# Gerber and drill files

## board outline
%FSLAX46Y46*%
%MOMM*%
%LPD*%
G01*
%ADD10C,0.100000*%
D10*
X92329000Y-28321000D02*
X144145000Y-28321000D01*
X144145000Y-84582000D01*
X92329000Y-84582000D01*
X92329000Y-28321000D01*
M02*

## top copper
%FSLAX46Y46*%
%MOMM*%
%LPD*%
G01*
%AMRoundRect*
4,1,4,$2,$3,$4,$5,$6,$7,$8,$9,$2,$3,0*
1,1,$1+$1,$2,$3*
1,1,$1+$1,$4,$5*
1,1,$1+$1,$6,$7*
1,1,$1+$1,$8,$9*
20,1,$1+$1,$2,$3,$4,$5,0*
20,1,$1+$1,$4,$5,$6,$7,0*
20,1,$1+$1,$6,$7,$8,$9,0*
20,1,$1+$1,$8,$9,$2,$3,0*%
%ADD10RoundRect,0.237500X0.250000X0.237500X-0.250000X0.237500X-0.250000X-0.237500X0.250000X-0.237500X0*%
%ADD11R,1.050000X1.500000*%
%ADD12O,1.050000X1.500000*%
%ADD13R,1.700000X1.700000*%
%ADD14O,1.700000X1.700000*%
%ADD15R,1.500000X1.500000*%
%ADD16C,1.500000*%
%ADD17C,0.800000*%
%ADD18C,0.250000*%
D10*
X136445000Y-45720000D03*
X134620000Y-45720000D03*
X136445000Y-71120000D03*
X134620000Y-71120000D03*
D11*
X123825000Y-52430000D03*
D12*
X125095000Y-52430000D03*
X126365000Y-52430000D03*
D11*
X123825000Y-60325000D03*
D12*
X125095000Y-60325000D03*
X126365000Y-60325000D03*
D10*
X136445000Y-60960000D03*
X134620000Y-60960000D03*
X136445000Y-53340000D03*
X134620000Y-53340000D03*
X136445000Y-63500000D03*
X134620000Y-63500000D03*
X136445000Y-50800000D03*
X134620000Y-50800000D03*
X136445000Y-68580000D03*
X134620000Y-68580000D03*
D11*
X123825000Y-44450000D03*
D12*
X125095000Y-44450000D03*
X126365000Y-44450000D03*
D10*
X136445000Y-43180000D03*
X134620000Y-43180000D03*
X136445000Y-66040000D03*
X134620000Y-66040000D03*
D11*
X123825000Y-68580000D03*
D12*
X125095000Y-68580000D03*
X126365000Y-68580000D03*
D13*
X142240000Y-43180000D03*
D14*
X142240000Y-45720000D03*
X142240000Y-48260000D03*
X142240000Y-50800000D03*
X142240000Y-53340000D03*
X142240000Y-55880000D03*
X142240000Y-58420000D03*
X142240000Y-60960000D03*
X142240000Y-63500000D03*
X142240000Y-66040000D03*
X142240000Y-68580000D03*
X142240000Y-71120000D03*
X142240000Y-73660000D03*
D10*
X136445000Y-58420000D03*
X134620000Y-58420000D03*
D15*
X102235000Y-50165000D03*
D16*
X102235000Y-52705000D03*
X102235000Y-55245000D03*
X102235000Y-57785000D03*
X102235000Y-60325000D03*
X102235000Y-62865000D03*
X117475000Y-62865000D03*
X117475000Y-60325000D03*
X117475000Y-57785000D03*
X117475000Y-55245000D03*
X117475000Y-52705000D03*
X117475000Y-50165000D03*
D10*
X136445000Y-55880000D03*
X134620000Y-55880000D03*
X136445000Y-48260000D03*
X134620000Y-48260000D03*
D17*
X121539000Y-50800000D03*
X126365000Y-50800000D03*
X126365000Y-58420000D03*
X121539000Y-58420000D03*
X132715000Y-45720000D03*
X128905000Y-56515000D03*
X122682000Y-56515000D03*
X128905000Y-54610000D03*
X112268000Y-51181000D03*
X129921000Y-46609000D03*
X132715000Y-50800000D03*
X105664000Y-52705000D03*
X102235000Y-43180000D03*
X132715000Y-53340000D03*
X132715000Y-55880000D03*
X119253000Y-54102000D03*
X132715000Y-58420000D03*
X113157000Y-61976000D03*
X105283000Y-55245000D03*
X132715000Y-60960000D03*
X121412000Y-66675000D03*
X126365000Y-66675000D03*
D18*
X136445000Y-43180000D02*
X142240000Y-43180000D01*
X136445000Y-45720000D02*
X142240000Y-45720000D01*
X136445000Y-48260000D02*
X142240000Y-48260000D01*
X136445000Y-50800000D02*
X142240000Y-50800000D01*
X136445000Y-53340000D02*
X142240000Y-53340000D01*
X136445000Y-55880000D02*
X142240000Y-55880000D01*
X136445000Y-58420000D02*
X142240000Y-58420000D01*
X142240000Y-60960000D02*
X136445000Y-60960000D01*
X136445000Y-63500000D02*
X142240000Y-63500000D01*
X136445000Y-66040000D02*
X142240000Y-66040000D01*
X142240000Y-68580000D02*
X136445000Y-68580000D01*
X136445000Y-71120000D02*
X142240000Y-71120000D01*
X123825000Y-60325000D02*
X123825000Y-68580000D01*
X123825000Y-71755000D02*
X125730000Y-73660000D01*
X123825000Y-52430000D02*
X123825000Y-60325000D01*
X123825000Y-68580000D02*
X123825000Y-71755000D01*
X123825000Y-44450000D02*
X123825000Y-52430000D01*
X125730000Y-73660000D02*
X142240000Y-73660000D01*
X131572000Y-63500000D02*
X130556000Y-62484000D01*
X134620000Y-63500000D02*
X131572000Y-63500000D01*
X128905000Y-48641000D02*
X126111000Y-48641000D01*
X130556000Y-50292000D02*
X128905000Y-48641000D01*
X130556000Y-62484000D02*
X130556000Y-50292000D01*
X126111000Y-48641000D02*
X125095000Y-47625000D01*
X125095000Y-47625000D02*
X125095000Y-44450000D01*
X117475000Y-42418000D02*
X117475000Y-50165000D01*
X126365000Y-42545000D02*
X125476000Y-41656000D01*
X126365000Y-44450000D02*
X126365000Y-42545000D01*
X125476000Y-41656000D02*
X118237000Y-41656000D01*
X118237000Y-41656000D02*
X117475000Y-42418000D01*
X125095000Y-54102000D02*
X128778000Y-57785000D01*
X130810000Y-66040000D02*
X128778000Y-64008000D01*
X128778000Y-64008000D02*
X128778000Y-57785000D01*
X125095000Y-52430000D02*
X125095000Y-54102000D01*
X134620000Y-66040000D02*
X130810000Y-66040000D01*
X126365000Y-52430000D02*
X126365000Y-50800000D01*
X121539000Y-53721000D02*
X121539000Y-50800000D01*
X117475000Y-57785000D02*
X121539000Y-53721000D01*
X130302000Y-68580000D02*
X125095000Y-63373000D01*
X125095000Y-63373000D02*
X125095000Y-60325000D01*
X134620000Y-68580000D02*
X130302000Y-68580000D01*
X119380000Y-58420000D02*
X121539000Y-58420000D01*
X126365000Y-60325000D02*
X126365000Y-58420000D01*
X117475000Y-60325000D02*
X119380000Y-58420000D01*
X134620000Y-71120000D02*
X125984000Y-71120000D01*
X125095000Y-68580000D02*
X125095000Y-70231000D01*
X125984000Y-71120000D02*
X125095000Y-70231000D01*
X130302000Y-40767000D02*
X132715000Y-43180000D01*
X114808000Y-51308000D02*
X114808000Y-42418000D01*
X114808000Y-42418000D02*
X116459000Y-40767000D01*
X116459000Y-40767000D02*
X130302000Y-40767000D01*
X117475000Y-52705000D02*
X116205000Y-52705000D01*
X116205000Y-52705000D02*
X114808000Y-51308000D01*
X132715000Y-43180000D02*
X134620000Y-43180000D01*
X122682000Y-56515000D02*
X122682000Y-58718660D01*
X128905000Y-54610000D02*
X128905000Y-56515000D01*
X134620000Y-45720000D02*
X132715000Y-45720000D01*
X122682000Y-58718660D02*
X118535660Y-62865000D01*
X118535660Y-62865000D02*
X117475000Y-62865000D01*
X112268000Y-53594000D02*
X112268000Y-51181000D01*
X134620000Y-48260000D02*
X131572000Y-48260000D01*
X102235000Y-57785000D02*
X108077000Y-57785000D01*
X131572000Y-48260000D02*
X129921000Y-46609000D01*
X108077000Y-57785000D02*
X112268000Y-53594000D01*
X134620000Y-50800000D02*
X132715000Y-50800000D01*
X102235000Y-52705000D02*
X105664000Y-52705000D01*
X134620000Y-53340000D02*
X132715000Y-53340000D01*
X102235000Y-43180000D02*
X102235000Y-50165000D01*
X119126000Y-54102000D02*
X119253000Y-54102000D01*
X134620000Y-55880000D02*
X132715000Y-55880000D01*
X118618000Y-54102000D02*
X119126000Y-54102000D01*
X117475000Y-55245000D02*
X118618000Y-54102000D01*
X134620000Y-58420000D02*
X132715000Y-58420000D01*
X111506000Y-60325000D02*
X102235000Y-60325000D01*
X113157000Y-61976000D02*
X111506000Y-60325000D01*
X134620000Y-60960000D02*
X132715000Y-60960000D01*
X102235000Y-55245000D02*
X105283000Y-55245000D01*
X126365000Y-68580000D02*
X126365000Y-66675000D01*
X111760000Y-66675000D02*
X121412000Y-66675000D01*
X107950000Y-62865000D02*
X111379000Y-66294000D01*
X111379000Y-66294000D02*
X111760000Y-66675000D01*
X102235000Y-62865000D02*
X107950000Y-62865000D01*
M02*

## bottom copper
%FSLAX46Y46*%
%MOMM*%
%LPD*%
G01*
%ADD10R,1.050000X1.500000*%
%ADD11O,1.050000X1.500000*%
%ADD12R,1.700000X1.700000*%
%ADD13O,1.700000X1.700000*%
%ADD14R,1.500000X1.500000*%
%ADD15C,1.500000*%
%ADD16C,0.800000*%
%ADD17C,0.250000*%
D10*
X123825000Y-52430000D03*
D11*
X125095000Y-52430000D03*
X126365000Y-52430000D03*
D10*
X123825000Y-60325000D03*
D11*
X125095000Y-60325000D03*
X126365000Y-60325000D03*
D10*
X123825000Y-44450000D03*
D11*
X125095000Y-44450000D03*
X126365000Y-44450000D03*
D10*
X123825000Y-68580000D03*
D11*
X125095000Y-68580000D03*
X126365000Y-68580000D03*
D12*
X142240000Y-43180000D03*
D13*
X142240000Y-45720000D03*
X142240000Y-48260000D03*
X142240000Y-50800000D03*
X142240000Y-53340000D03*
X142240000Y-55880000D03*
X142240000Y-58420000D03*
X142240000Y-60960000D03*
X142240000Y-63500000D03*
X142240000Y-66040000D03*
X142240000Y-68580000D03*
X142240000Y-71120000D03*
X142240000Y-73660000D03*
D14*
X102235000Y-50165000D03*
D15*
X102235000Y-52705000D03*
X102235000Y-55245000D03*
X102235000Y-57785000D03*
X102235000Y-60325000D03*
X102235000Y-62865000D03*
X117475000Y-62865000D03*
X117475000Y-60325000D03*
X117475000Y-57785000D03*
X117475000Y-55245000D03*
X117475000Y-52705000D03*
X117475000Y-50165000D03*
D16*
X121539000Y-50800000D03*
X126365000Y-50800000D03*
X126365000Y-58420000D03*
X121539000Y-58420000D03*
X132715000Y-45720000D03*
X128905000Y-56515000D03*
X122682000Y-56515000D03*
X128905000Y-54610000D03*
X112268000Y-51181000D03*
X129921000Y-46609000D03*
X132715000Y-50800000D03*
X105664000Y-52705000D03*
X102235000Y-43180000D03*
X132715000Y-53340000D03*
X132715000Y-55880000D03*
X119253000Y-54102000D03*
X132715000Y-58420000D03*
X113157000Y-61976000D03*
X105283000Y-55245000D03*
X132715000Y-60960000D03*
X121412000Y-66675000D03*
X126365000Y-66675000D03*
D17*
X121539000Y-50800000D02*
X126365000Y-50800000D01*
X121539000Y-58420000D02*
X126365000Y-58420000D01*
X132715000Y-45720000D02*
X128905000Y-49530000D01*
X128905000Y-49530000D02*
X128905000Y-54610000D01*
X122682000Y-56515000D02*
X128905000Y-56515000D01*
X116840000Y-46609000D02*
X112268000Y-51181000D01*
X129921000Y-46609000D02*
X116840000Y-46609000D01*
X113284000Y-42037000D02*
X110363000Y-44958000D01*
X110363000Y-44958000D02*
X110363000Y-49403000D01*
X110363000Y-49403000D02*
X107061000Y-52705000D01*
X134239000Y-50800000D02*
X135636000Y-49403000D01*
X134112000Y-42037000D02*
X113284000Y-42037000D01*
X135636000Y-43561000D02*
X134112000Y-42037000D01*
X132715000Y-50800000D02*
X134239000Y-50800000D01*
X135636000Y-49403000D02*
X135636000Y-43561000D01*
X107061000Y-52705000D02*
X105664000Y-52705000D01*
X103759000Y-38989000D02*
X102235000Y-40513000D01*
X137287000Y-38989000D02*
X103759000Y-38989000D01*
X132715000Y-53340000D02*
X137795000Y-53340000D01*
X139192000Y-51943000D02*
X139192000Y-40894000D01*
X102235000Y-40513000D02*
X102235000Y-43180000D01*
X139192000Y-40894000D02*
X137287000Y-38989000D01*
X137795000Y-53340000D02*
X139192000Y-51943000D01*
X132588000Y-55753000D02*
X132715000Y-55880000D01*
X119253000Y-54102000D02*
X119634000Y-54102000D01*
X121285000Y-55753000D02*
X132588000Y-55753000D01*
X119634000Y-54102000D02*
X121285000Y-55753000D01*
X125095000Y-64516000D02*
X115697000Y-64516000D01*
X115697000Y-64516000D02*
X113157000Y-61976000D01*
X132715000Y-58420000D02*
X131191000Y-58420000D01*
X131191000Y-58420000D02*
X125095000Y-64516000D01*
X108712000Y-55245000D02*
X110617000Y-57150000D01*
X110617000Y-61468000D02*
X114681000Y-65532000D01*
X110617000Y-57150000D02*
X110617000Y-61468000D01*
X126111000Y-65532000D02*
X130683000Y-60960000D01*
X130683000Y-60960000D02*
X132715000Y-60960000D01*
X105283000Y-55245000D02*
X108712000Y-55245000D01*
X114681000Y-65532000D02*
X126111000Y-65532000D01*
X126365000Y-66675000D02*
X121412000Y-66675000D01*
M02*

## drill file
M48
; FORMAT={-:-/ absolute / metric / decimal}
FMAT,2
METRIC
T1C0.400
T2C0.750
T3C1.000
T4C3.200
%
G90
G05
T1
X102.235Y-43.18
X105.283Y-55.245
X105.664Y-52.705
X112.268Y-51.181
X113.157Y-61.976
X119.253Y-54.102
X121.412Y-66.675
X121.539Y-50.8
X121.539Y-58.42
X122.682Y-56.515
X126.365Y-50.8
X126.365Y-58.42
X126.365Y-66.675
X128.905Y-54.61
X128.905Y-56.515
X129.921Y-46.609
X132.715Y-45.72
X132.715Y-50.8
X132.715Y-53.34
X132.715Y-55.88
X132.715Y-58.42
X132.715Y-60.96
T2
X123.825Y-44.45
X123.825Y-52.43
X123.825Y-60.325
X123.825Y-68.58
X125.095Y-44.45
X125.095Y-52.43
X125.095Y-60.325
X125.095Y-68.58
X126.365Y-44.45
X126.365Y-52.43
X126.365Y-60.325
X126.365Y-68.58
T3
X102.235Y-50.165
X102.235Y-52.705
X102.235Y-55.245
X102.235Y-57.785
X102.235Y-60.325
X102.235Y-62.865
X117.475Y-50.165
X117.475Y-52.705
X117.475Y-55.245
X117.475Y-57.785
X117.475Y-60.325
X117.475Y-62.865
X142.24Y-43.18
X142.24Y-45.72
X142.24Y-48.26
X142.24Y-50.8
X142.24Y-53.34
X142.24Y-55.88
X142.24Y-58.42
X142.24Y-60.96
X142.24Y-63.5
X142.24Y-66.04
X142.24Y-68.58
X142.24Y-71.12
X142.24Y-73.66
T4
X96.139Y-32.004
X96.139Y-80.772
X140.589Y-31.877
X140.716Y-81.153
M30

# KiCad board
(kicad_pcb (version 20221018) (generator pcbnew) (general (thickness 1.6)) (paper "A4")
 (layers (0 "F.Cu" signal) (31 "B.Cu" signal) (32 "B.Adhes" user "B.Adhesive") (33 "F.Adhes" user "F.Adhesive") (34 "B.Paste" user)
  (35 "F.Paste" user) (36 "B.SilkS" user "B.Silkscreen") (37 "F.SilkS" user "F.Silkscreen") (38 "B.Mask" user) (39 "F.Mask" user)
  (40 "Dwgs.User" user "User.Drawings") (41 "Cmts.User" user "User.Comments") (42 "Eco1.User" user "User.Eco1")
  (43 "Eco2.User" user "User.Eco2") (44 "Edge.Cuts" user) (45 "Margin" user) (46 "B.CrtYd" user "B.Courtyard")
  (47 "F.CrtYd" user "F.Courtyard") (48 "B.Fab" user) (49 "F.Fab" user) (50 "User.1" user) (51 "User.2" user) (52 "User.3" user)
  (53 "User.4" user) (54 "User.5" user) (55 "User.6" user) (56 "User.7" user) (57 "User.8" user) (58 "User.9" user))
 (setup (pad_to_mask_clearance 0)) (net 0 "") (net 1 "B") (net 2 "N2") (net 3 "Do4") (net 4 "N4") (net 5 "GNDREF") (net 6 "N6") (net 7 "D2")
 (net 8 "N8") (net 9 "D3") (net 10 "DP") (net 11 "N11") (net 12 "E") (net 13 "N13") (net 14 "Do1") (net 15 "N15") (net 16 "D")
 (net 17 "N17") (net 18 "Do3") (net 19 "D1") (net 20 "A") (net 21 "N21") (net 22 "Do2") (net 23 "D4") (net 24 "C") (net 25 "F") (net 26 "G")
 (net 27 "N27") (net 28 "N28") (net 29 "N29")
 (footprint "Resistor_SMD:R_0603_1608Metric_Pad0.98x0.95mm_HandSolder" (layer "F.Cu") (at 135.5325 45.72 180)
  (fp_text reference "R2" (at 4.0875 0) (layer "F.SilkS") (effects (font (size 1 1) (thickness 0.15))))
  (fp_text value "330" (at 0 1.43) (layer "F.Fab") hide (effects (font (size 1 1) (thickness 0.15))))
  (pad "1" smd roundrect (at -0.9125 0 180) (size 0.975 0.95) (layers "F.Cu" "F.Paste" "F.Mask") (roundrect_rratio 0.25) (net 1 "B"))
  (pad "2" smd roundrect (at 0.9125 0 180) (size 0.975 0.95) (layers "F.Cu" "F.Paste" "F.Mask") (roundrect_rratio 0.25) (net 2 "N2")))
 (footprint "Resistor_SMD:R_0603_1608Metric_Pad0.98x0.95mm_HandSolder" (layer "F.Cu") (at 135.5325 71.12 180)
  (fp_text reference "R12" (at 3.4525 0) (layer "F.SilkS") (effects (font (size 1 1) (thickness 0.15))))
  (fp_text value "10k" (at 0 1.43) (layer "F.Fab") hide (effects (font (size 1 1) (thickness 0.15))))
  (pad "1" smd roundrect (at -0.9125 0 180) (size 0.975 0.95) (layers "F.Cu" "F.Paste" "F.Mask") (roundrect_rratio 0.25) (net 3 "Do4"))
  (pad "2" smd roundrect (at 0.9125 0 180) (size 0.975 0.95) (layers "F.Cu" "F.Paste" "F.Mask") (roundrect_rratio 0.25) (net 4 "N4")))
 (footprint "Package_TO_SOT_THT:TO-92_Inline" (layer "F.Cu") (at 123.825 52.43)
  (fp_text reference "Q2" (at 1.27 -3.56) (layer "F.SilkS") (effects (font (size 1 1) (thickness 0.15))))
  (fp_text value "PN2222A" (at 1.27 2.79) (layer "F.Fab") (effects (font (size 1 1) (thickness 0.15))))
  (pad "1" thru_hole rect (at 0 0) (size 1.05 1.5) (drill 0.75) (layers "*.Cu" "*.Mask") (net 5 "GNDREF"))
  (pad "2" thru_hole oval (at 1.27 0) (size 1.05 1.5) (drill 0.75) (layers "*.Cu" "*.Mask") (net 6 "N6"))
  (pad "3" thru_hole oval (at 2.54 0) (size 1.05 1.5) (drill 0.75) (layers "*.Cu" "*.Mask") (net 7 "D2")))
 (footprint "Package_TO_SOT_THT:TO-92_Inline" (layer "F.Cu") (at 123.825 60.325)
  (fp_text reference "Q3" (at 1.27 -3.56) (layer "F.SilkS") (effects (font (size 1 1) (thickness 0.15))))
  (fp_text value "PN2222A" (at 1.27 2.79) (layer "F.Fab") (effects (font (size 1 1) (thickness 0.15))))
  (pad "1" thru_hole rect (at 0 0) (size 1.05 1.5) (drill 0.75) (layers "*.Cu" "*.Mask") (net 5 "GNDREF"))
  (pad "2" thru_hole oval (at 1.27 0) (size 1.05 1.5) (drill 0.75) (layers "*.Cu" "*.Mask") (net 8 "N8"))
  (pad "3" thru_hole oval (at 2.54 0) (size 1.05 1.5) (drill 0.75) (layers "*.Cu" "*.Mask") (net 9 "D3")))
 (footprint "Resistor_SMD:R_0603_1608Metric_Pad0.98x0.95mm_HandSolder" (layer "F.Cu") (at 135.5325 60.96 180)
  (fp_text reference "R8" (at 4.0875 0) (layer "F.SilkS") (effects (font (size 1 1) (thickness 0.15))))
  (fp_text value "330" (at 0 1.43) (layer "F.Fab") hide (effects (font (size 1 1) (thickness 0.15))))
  (pad "1" smd roundrect (at -0.9125 0 180) (size 0.975 0.95) (layers "F.Cu" "F.Paste" "F.Mask") (roundrect_rratio 0.25) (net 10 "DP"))
  (pad "2" smd roundrect (at 0.9125 0 180) (size 0.975 0.95) (layers "F.Cu" "F.Paste" "F.Mask") (roundrect_rratio 0.25) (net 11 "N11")))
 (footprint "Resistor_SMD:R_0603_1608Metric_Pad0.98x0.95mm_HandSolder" (layer "F.Cu") (at 135.5325 53.34 180)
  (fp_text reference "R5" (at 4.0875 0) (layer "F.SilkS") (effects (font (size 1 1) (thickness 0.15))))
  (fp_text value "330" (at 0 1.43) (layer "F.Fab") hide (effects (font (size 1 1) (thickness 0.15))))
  (pad "1" smd roundrect (at -0.9125 0 180) (size 0.975 0.95) (layers "F.Cu" "F.Paste" "F.Mask") (roundrect_rratio 0.25) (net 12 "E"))
  (pad "2" smd roundrect (at 0.9125 0 180) (size 0.975 0.95) (layers "F.Cu" "F.Paste" "F.Mask") (roundrect_rratio 0.25) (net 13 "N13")))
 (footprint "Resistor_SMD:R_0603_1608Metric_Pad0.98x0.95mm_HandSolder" (layer "F.Cu") (at 135.5325 63.5 180)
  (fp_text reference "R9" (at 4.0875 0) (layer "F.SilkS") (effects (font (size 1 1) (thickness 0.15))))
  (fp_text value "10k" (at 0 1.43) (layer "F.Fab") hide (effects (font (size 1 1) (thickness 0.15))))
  (pad "1" smd roundrect (at -0.9125 0 180) (size 0.975 0.95) (layers "F.Cu" "F.Paste" "F.Mask") (roundrect_rratio 0.25) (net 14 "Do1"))
  (pad "2" smd roundrect (at 0.9125 0 180) (size 0.975 0.95) (layers "F.Cu" "F.Paste" "F.Mask") (roundrect_rratio 0.25) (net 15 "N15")))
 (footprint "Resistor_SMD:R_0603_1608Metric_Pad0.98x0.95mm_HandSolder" (layer "F.Cu") (at 135.5325 50.8 180)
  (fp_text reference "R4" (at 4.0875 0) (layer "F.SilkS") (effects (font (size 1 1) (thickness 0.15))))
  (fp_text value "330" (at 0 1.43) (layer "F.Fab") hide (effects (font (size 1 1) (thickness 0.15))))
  (pad "1" smd roundrect (at -0.9125 0 180) (size 0.975 0.95) (layers "F.Cu" "F.Paste" "F.Mask") (roundrect_rratio 0.25) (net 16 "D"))
  (pad "2" smd roundrect (at 0.9125 0 180) (size 0.975 0.95) (layers "F.Cu" "F.Paste" "F.Mask") (roundrect_rratio 0.25) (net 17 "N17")))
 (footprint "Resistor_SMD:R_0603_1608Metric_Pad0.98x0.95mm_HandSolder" (layer "F.Cu") (at 135.5325 68.58 180)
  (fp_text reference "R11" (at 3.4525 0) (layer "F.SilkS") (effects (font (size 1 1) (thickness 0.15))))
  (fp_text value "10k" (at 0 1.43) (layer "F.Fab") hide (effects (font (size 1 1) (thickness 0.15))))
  (pad "1" smd roundrect (at -0.9125 0 180) (size 0.975 0.95) (layers "F.Cu" "F.Paste" "F.Mask") (roundrect_rratio 0.25) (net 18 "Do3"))
  (pad "2" smd roundrect (at 0.9125 0 180) (size 0.975 0.95) (layers "F.Cu" "F.Paste" "F.Mask") (roundrect_rratio 0.25) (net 8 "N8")))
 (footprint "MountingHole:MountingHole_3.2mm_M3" (layer "F.Cu") (at 96.139 32.004)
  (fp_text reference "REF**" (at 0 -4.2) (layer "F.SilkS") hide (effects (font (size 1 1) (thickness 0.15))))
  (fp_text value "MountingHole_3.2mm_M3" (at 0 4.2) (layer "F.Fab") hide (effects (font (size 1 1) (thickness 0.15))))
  (pad "" np_thru_hole circle (at 0 0) (size 3.2 3.2) (drill 3.2) (layers "*.Cu" "*.Mask")))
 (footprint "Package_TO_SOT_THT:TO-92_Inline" (layer "F.Cu") (at 123.825 44.45)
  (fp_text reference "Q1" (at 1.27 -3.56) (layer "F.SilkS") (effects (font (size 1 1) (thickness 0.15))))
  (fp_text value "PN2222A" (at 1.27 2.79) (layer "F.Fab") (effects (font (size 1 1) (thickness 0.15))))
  (pad "1" thru_hole rect (at 0 0) (size 1.05 1.5) (drill 0.75) (layers "*.Cu" "*.Mask") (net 5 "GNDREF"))
  (pad "2" thru_hole oval (at 1.27 0) (size 1.05 1.5) (drill 0.75) (layers "*.Cu" "*.Mask") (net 15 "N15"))
  (pad "3" thru_hole oval (at 2.54 0) (size 1.05 1.5) (drill 0.75) (layers "*.Cu" "*.Mask") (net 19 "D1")))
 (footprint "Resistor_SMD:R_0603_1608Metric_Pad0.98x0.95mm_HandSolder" (layer "F.Cu") (at 135.5325 43.18 180)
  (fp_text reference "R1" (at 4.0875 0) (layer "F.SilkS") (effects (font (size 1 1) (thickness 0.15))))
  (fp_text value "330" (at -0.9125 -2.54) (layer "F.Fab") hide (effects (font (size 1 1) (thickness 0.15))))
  (pad "1" smd roundrect (at -0.9125 0 180) (size 0.975 0.95) (layers "F.Cu" "F.Paste" "F.Mask") (roundrect_rratio 0.25) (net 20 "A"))
  (pad "2" smd roundrect (at 0.9125 0 180) (size 0.975 0.95) (layers "F.Cu" "F.Paste" "F.Mask") (roundrect_rratio 0.25) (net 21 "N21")))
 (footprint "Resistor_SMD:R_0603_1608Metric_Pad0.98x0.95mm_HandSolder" (layer "F.Cu") (at 135.5325 66.04 180)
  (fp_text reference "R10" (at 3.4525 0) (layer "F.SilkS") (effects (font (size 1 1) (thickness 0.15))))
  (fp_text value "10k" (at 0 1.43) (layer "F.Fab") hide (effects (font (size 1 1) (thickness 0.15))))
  (pad "1" smd roundrect (at -0.9125 0 180) (size 0.975 0.95) (layers "F.Cu" "F.Paste" "F.Mask") (roundrect_rratio 0.25) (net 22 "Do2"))
  (pad "2" smd roundrect (at 0.9125 0 180) (size 0.975 0.95) (layers "F.Cu" "F.Paste" "F.Mask") (roundrect_rratio 0.25) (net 6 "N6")))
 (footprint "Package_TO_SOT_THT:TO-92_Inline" (layer "F.Cu") (at 123.825 68.58)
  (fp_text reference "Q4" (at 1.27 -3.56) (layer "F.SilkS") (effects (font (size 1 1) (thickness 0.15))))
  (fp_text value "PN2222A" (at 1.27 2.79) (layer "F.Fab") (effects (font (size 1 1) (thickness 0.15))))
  (pad "1" thru_hole rect (at 0 0) (size 1.05 1.5) (drill 0.75) (layers "*.Cu" "*.Mask") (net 5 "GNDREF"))
  (pad "2" thru_hole oval (at 1.27 0) (size 1.05 1.5) (drill 0.75) (layers "*.Cu" "*.Mask") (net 4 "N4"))
  (pad "3" thru_hole oval (at 2.54 0) (size 1.05 1.5) (drill 0.75) (layers "*.Cu" "*.Mask") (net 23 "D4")))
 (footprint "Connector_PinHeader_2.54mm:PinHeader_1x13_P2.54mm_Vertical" (layer "F.Cu") (at 142.24 43.18)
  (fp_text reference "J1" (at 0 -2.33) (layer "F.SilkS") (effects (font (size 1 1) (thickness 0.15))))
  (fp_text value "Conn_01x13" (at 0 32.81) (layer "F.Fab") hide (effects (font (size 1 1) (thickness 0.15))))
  (pad "1" thru_hole rect (at 0 0) (size 1.7 1.7) (drill 1) (layers "*.Cu" "*.Mask") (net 20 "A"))
  (pad "2" thru_hole oval (at 0 2.54) (size 1.7 1.7) (drill 1) (layers "*.Cu" "*.Mask") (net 1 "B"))
  (pad "3" thru_hole oval (at 0 5.08) (size 1.7 1.7) (drill 1) (layers "*.Cu" "*.Mask") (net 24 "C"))
  (pad "4" thru_hole oval (at 0 7.62) (size 1.7 1.7) (drill 1) (layers "*.Cu" "*.Mask") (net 16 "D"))
  (pad "5" thru_hole oval (at 0 10.16) (size 1.7 1.7) (drill 1) (layers "*.Cu" "*.Mask") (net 12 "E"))
  (pad "6" thru_hole oval (at 0 12.7) (size 1.7 1.7) (drill 1) (layers "*.Cu" "*.Mask") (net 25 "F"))
  (pad "7" thru_hole oval (at 0 15.24) (size 1.7 1.7) (drill 1) (layers "*.Cu" "*.Mask") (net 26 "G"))
  (pad "8" thru_hole oval (at 0 17.78) (size 1.7 1.7) (drill 1) (layers "*.Cu" "*.Mask") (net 10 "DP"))
  (pad "9" thru_hole oval (at 0 20.32) (size 1.7 1.7) (drill 1) (layers "*.Cu" "*.Mask") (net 14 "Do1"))
  (pad "10" thru_hole oval (at 0 22.86) (size 1.7 1.7) (drill 1) (layers "*.Cu" "*.Mask") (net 22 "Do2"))
  (pad "11" thru_hole oval (at 0 25.4) (size 1.7 1.7) (drill 1) (layers "*.Cu" "*.Mask") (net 18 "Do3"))
  (pad "12" thru_hole oval (at 0 27.94) (size 1.7 1.7) (drill 1) (layers "*.Cu" "*.Mask") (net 3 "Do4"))
  (pad "13" thru_hole oval (at 0 30.48) (size 1.7 1.7) (drill 1) (layers "*.Cu" "*.Mask") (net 5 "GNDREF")))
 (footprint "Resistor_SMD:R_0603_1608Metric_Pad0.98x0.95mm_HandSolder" (layer "F.Cu") (at 135.5325 58.42 180)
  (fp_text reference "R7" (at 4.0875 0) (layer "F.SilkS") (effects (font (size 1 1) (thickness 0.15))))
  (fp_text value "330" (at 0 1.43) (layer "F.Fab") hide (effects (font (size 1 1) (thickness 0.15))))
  (pad "1" smd roundrect (at -0.9125 0 180) (size 0.975 0.95) (layers "F.Cu" "F.Paste" "F.Mask") (roundrect_rratio 0.25) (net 26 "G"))
  (pad "2" smd roundrect (at 0.9125 0 180) (size 0.975 0.95) (layers "F.Cu" "F.Paste" "F.Mask") (roundrect_rratio 0.25) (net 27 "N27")))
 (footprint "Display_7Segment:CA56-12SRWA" (layer "F.Cu") (at 102.235 50.165)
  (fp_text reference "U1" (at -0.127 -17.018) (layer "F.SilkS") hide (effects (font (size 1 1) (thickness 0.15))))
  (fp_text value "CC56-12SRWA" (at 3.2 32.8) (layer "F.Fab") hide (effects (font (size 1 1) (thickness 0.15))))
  (pad "1" thru_hole rect (at 0 0) (size 1.5 1.5) (drill 1) (layers "*.Cu" "*.Mask") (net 13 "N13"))
  (pad "2" thru_hole circle (at 0 2.54) (size 1.5 1.5) (drill 1) (layers "*.Cu" "*.Mask") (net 17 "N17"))
  (pad "3" thru_hole circle (at 0 5.08) (size 1.5 1.5) (drill 1) (layers "*.Cu" "*.Mask") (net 11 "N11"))
  (pad "4" thru_hole circle (at 0 7.62) (size 1.5 1.5) (drill 1) (layers "*.Cu" "*.Mask") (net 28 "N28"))
  (pad "5" thru_hole circle (at 0 10.16) (size 1.5 1.5) (drill 1) (layers "*.Cu" "*.Mask") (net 27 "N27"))
  (pad "6" thru_hole circle (at 0 12.7) (size 1.5 1.5) (drill 1) (layers "*.Cu" "*.Mask") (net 23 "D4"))
  (pad "7" thru_hole circle (at 15.24 12.7) (size 1.5 1.5) (drill 1) (layers "*.Cu" "*.Mask") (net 2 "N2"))
  (pad "8" thru_hole circle (at 15.24 10.16) (size 1.5 1.5) (drill 1) (layers "*.Cu" "*.Mask") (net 9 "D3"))
  (pad "9" thru_hole circle (at 15.24 7.62) (size 1.5 1.5) (drill 1) (layers "*.Cu" "*.Mask") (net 7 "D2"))
  (pad "10" thru_hole circle (at 15.24 5.08) (size 1.5 1.5) (drill 1) (layers "*.Cu" "*.Mask") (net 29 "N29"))
  (pad "11" thru_hole circle (at 15.24 2.54) (size 1.5 1.5) (drill 1) (layers "*.Cu" "*.Mask") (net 21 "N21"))
  (pad "12" thru_hole circle (at 15.24 0) (size 1.5 1.5) (drill 1) (layers "*.Cu" "*.Mask") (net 19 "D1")))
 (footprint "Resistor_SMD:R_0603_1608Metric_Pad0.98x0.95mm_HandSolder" (layer "F.Cu") (at 135.5325 55.88 180)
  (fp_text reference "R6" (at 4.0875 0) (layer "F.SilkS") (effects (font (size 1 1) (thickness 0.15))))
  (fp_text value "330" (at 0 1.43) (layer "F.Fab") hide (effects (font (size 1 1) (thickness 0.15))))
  (pad "1" smd roundrect (at -0.9125 0 180) (size 0.975 0.95) (layers "F.Cu" "F.Paste" "F.Mask") (roundrect_rratio 0.25) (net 25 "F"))
  (pad "2" smd roundrect (at 0.9125 0 180) (size 0.975 0.95) (layers "F.Cu" "F.Paste" "F.Mask") (roundrect_rratio 0.25) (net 29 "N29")))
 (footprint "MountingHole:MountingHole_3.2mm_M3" (layer "F.Cu") (at 140.589 31.877)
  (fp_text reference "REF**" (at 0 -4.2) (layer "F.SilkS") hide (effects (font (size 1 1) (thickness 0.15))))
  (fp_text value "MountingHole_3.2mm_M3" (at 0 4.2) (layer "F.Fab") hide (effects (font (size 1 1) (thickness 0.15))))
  (pad "" np_thru_hole circle (at 0 0) (size 3.2 3.2) (drill 3.2) (layers "*.Cu" "*.Mask")))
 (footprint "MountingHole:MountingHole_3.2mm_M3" (layer "F.Cu") (at 140.716 81.153)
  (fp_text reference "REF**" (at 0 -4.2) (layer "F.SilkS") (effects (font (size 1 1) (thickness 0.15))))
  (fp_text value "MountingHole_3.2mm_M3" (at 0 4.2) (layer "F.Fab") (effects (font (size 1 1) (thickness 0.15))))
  (pad "" np_thru_hole circle (at 0 0) (size 3.2 3.2) (drill 3.2) (layers "*.Cu" "*.Mask")))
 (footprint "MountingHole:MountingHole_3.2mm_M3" (layer "F.Cu") (at 96.139 80.772)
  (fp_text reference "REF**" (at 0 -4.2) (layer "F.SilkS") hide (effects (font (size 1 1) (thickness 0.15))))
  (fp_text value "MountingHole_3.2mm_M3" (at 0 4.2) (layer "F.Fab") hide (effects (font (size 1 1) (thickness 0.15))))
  (pad "" np_thru_hole circle (at 0 0) (size 3.2 3.2) (drill 3.2) (layers "*.Cu" "*.Mask")))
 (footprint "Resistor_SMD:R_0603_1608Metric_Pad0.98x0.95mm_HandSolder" (layer "F.Cu") (at 135.5325 48.26 180)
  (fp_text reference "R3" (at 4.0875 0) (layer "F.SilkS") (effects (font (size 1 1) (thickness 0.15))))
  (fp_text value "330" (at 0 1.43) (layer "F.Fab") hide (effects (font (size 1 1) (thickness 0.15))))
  (pad "1" smd roundrect (at -0.9125 0 180) (size 0.975 0.95) (layers "F.Cu" "F.Paste" "F.Mask") (roundrect_rratio 0.25) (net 24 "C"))
  (pad "2" smd roundrect (at 0.9125 0 180) (size 0.975 0.95) (layers "F.Cu" "F.Paste" "F.Mask") (roundrect_rratio 0.25) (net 28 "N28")))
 (gr_rect (start 92.329 28.321) (end 144.145 84.582) (stroke (width 0.1) (type default)) (fill none) (layer "Edge.Cuts"))
 (segment (start 136.445 43.18) (end 142.24 43.18) (width 0.25) (layer "F.Cu") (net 20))
 (segment (start 136.445 45.72) (end 142.24 45.72) (width 0.25) (layer "F.Cu") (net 1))
 (segment (start 136.445 48.26) (end 142.24 48.26) (width 0.25) (layer "F.Cu") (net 24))
 (segment (start 136.445 50.8) (end 142.24 50.8) (width 0.25) (layer "F.Cu") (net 16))
 (segment (start 136.445 53.34) (end 142.24 53.34) (width 0.25) (layer "F.Cu") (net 12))
 (segment (start 136.445 55.88) (end 142.24 55.88) (width 0.25) (layer "F.Cu") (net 25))
 (segment (start 136.445 58.42) (end 142.24 58.42) (width 0.25) (layer "F.Cu") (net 26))
 (segment (start 142.24 60.96) (end 136.445 60.96) (width 0.25) (layer "F.Cu") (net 10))
 (segment (start 136.445 63.5) (end 142.24 63.5) (width 0.25) (layer "F.Cu") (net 14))
 (segment (start 136.445 66.04) (end 142.24 66.04) (width 0.25) (layer "F.Cu") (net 22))
 (segment (start 142.24 68.58) (end 136.445 68.58) (width 0.25) (layer "F.Cu") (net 18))
 (segment (start 136.445 71.12) (end 142.24 71.12) (width 0.25) (layer "F.Cu") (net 3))
 (segment (start 123.825 60.325) (end 123.825 68.58) (width 0.25) (layer "F.Cu") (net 5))
 (segment (start 123.825 71.755) (end 125.73 73.66) (width 0.25) (layer "F.Cu") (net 5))
 (segment (start 123.825 52.43) (end 123.825 60.325) (width 0.25) (layer "F.Cu") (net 5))
 (segment (start 123.825 68.58) (end 123.825 71.755) (width 0.25) (layer "F.Cu") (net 5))
 (segment (start 123.825 44.45) (end 123.825 52.43) (width 0.25) (layer "F.Cu") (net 5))
 (segment (start 125.73 73.66) (end 142.24 73.66) (width 0.25) (layer "F.Cu") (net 5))
 (segment (start 131.572 63.5) (end 130.556 62.484) (width 0.25) (layer "F.Cu") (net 15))
 (segment (start 134.62 63.5) (end 131.572 63.5) (width 0.25) (layer "F.Cu") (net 15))
 (segment (start 128.905 48.641) (end 126.111 48.641) (width 0.25) (layer "F.Cu") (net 15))
 (segment (start 130.556 50.292) (end 128.905 48.641) (width 0.25) (layer "F.Cu") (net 15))
 (segment (start 130.556 62.484) (end 130.556 50.292) (width 0.25) (layer "F.Cu") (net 15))
 (segment (start 126.111 48.641) (end 125.095 47.625) (width 0.25) (layer "F.Cu") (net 15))
 (segment (start 125.095 47.625) (end 125.095 44.45) (width 0.25) (layer "F.Cu") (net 15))
 (segment (start 117.475 42.418) (end 117.475 50.165) (width 0.25) (layer "F.Cu") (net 19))
 (segment (start 126.365 42.545) (end 125.476 41.656) (width 0.25) (layer "F.Cu") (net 19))
 (segment (start 126.365 44.45) (end 126.365 42.545) (width 0.25) (layer "F.Cu") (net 19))
 (segment (start 125.476 41.656) (end 118.237 41.656) (width 0.25) (layer "F.Cu") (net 19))
 (segment (start 118.237 41.656) (end 117.475 42.418) (width 0.25) (layer "F.Cu") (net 19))
 (segment (start 125.095 54.102) (end 128.778 57.785) (width 0.25) (layer "F.Cu") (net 6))
 (segment (start 130.81 66.04) (end 128.778 64.008) (width 0.25) (layer "F.Cu") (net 6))
 (segment (start 128.778 64.008) (end 128.778 57.785) (width 0.25) (layer "F.Cu") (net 6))
 (segment (start 125.095 52.43) (end 125.095 54.102) (width 0.25) (layer "F.Cu") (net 6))
 (segment (start 134.62 66.04) (end 130.81 66.04) (width 0.25) (layer "F.Cu") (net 6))
 (segment (start 126.365 52.43) (end 126.365 50.8) (width 0.25) (layer "F.Cu") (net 7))
 (segment (start 121.539 53.721) (end 121.539 50.8) (width 0.25) (layer "F.Cu") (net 7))
 (segment (start 117.475 57.785) (end 121.539 53.721) (width 0.25) (layer "F.Cu") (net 7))
 (via (at 121.539 50.8) (size 0.8) (drill 0.4) (layers "F.Cu" "B.Cu") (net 7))
 (via (at 126.365 50.8) (size 0.8) (drill 0.4) (layers "F.Cu" "B.Cu") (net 7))
 (segment (start 121.539 50.8) (end 126.365 50.8) (width 0.25) (layer "B.Cu") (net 7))
 (segment (start 130.302 68.58) (end 125.095 63.373) (width 0.25) (layer "F.Cu") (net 8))
 (segment (start 125.095 63.373) (end 125.095 60.325) (width 0.25) (layer "F.Cu") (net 8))
 (segment (start 134.62 68.58) (end 130.302 68.58) (width 0.25) (layer "F.Cu") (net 8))
 (segment (start 119.38 58.42) (end 121.539 58.42) (width 0.25) (layer "F.Cu") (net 9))
 (segment (start 126.365 60.325) (end 126.365 58.42) (width 0.25) (layer "F.Cu") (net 9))
 (segment (start 117.475 60.325) (end 119.38 58.42) (width 0.25) (layer "F.Cu") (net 9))
 (via (at 126.365 58.42) (size 0.8) (drill 0.4) (layers "F.Cu" "B.Cu") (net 9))
 (via (at 121.539 58.42) (size 0.8) (drill 0.4) (layers "F.Cu" "B.Cu") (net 9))
 (segment (start 121.539 58.42) (end 126.365 58.42) (width 0.25) (layer "B.Cu") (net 9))
 (segment (start 134.62 71.12) (end 125.984 71.12) (width 0.25) (layer "F.Cu") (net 4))
 (segment (start 125.095 68.58) (end 125.095 70.231) (width 0.25) (layer "F.Cu") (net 4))
 (segment (start 125.984 71.12) (end 125.095 70.231) (width 0.25) (layer "F.Cu") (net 4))
 (segment (start 130.302 40.767) (end 132.715 43.18) (width 0.25) (layer "F.Cu") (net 21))
 (segment (start 114.808 51.308) (end 114.808 42.418) (width 0.25) (layer "F.Cu") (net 21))
 (segment (start 114.808 42.418) (end 116.459 40.767) (width 0.25) (layer "F.Cu") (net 21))
 (segment (start 116.459 40.767) (end 130.302 40.767) (width 0.25) (layer "F.Cu") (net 21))
 (segment (start 117.475 52.705) (end 116.205 52.705) (width 0.25) (layer "F.Cu") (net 21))
 (segment (start 116.205 52.705) (end 114.808 51.308) (width 0.25) (layer "F.Cu") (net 21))
 (segment (start 132.715 43.18) (end 134.62 43.18) (width 0.25) (layer "F.Cu") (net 21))
 (segment (start 122.682 56.515) (end 122.682 58.71866) (width 0.25) (layer "F.Cu") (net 2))
 (segment (start 128.905 54.61) (end 128.905 56.515) (width 0.25) (layer "F.Cu") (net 2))
 (segment (start 134.62 45.72) (end 132.715 45.72) (width 0.25) (layer "F.Cu") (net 2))
 (segment (start 122.682 58.71866) (end 118.53566 62.865) (width 0.25) (layer "F.Cu") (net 2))
 (segment (start 118.53566 62.865) (end 117.475 62.865) (width 0.25) (layer "F.Cu") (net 2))
 (via (at 132.715 45.72) (size 0.8) (drill 0.4) (layers "F.Cu" "B.Cu") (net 2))
 (via (at 128.905 56.515) (size 0.8) (drill 0.4) (layers "F.Cu" "B.Cu") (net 2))
 (via (at 122.682 56.515) (size 0.8) (drill 0.4) (layers "F.Cu" "B.Cu") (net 2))
 (via (at 128.905 54.61) (size 0.8) (drill 0.4) (layers "F.Cu" "B.Cu") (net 2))
 (segment (start 132.715 45.72) (end 128.905 49.53) (width 0.25) (layer "B.Cu") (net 2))
 (segment (start 128.905 49.53) (end 128.905 54.61) (width 0.25) (layer "B.Cu") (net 2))
 (segment (start 122.682 56.515) (end 128.905 56.515) (width 0.25) (layer "B.Cu") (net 2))
 (segment (start 112.268 53.594) (end 112.268 51.181) (width 0.25) (layer "F.Cu") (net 28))
 (segment (start 134.62 48.26) (end 131.572 48.26) (width 0.25) (layer "F.Cu") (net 28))
 (segment (start 102.235 57.785) (end 108.077 57.785) (width 0.25) (layer "F.Cu") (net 28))
 (segment (start 131.572 48.26) (end 129.921 46.609) (width 0.25) (layer "F.Cu") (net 28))
 (segment (start 108.077 57.785) (end 112.268 53.594) (width 0.25) (layer "F.Cu") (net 28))
 (via (at 112.268 51.181) (size 0.8) (drill 0.4) (layers "F.Cu" "B.Cu") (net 28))
 (via (at 129.921 46.609) (size 0.8) (drill 0.4) (layers "F.Cu" "B.Cu") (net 28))
 (segment (start 116.84 46.609) (end 112.268 51.181) (width 0.25) (layer "B.Cu") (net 28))
 (segment (start 129.921 46.609) (end 116.84 46.609) (width 0.25) (layer "B.Cu") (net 28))
 (segment (start 134.62 50.8) (end 132.715 50.8) (width 0.25) (layer "F.Cu") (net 17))
 (segment (start 102.235 52.705) (end 105.664 52.705) (width 0.25) (layer "F.Cu") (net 17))
 (via (at 132.715 50.8) (size 0.8) (drill 0.4) (layers "F.Cu" "B.Cu") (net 17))
 (via (at 105.664 52.705) (size 0.8) (drill 0.4) (layers "F.Cu" "B.Cu") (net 17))
 (segment (start 113.284 42.037) (end 110.363 44.958) (width 0.25) (layer "B.Cu") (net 17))
 (segment (start 110.363 44.958) (end 110.363 49.403) (width 0.25) (layer "B.Cu") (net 17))
 (segment (start 110.363 49.403) (end 107.061 52.705) (width 0.25) (layer "B.Cu") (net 17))
 (segment (start 134.239 50.8) (end 135.636 49.403) (width 0.25) (layer "B.Cu") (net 17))
 (segment (start 134.112 42.037) (end 113.284 42.037) (width 0.25) (layer "B.Cu") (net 17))
 (segment (start 135.636 43.561) (end 134.112 42.037) (width 0.25) (layer "B.Cu") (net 17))
 (segment (start 132.715 50.8) (end 134.239 50.8) (width 0.25) (layer "B.Cu") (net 17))
 (segment (start 135.636 49.403) (end 135.636 43.561) (width 0.25) (layer "B.Cu") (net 17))
 (segment (start 107.061 52.705) (end 105.664 52.705) (width 0.25) (layer "B.Cu") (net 17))
 (segment (start 134.62 53.34) (end 132.715 53.34) (width 0.25) (layer "F.Cu") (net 13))
 (segment (start 102.235 43.18) (end 102.235 50.165) (width 0.25) (layer "F.Cu") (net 13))
 (via (at 102.235 43.18) (size 0.8) (drill 0.4) (layers "F.Cu" "B.Cu") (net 13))
 (via (at 132.715 53.34) (size 0.8) (drill 0.4) (layers "F.Cu" "B.Cu") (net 13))
 (segment (start 103.759 38.989) (end 102.235 40.513) (width 0.25) (layer "B.Cu") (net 13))
 (segment (start 137.287 38.989) (end 103.759 38.989) (width 0.25) (layer "B.Cu") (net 13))
 (segment (start 132.715 53.34) (end 137.795 53.34) (width 0.25) (layer "B.Cu") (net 13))
 (segment (start 139.192 51.943) (end 139.192 40.894) (width 0.25) (layer "B.Cu") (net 13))
 (segment (start 102.235 40.513) (end 102.235 43.18) (width 0.25) (layer "B.Cu") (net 13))
 (segment (start 139.192 40.894) (end 137.287 38.989) (width 0.25) (layer "B.Cu") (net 13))
 (segment (start 137.795 53.34) (end 139.192 51.943) (width 0.25) (layer "B.Cu") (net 13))
 (segment (start 119.126 54.102) (end 119.253 54.102) (width 0.25) (layer "F.Cu") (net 29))
 (segment (start 134.62 55.88) (end 132.715 55.88) (width 0.25) (layer "F.Cu") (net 29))
 (segment (start 118.618 54.102) (end 119.126 54.102) (width 0.25) (layer "F.Cu") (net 29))
 (segment (start 117.475 55.245) (end 118.618 54.102) (width 0.25) (layer "F.Cu") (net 29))
 (via (at 132.715 55.88) (size 0.8) (drill 0.4) (layers "F.Cu" "B.Cu") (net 29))
 (via (at 119.253 54.102) (size 0.8) (drill 0.4) (layers "F.Cu" "B.Cu") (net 29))
 (segment (start 132.588 55.753) (end 132.715 55.88) (width 0.25) (layer "B.Cu") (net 29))
 (segment (start 119.253 54.102) (end 119.634 54.102) (width 0.25) (layer "B.Cu") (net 29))
 (segment (start 121.285 55.753) (end 132.588 55.753) (width 0.25) (layer "B.Cu") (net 29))
 (segment (start 119.634 54.102) (end 121.285 55.753) (width 0.25) (layer "B.Cu") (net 29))
 (segment (start 134.62 58.42) (end 132.715 58.42) (width 0.25) (layer "F.Cu") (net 27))
 (segment (start 111.506 60.325) (end 102.235 60.325) (width 0.25) (layer "F.Cu") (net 27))
 (segment (start 113.157 61.976) (end 111.506 60.325) (width 0.25) (layer "F.Cu") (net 27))
 (via (at 132.715 58.42) (size 0.8) (drill 0.4) (layers "F.Cu" "B.Cu") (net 27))
 (via (at 113.157 61.976) (size 0.8) (drill 0.4) (layers "F.Cu" "B.Cu") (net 27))
 (segment (start 125.095 64.516) (end 115.697 64.516) (width 0.25) (layer "B.Cu") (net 27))
 (segment (start 115.697 64.516) (end 113.157 61.976) (width 0.25) (layer "B.Cu") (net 27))
 (segment (start 132.715 58.42) (end 131.191 58.42) (width 0.25) (layer "B.Cu") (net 27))
 (segment (start 131.191 58.42) (end 125.095 64.516) (width 0.25) (layer "B.Cu") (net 27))
 (segment (start 134.62 60.96) (end 132.715 60.96) (width 0.25) (layer "F.Cu") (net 11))
 (segment (start 102.235 55.245) (end 105.283 55.245) (width 0.25) (layer "F.Cu") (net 11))
 (via (at 105.283 55.245) (size 0.8) (drill 0.4) (layers "F.Cu" "B.Cu") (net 11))
 (via (at 132.715 60.96) (size 0.8) (drill 0.4) (layers "F.Cu" "B.Cu") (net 11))
 (segment (start 108.712 55.245) (end 110.617 57.15) (width 0.25) (layer "B.Cu") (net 11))
 (segment (start 110.617 61.468) (end 114.681 65.532) (width 0.25) (layer "B.Cu") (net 11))
 (segment (start 110.617 57.15) (end 110.617 61.468) (width 0.25) (layer "B.Cu") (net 11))
 (segment (start 126.111 65.532) (end 130.683 60.96) (width 0.25) (layer "B.Cu") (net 11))
 (segment (start 130.683 60.96) (end 132.715 60.96) (width 0.25) (layer "B.Cu") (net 11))
 (segment (start 105.283 55.245) (end 108.712 55.245) (width 0.25) (layer "B.Cu") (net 11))
 (segment (start 114.681 65.532) (end 126.111 65.532) (width 0.25) (layer "B.Cu") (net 11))
 (segment (start 126.365 68.58) (end 126.365 66.675) (width 0.25) (layer "F.Cu") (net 23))
 (segment (start 111.76 66.675) (end 121.412 66.675) (width 0.25) (layer "F.Cu") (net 23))
 (segment (start 107.95 62.865) (end 111.379 66.294) (width 0.25) (layer "F.Cu") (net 23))
 (segment (start 111.379 66.294) (end 111.76 66.675) (width 0.25) (layer "F.Cu") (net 23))
 (segment (start 102.235 62.865) (end 107.95 62.865) (width 0.25) (layer "F.Cu") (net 23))
 (via (at 121.412 66.675) (size 0.8) (drill 0.4) (layers "F.Cu" "B.Cu") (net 23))
 (via (at 126.365 66.675) (size 0.8) (drill 0.4) (layers "F.Cu" "B.Cu") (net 23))
 (segment (start 126.365 66.675) (end 121.412 66.675) (width 0.25) (layer "B.Cu") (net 23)))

